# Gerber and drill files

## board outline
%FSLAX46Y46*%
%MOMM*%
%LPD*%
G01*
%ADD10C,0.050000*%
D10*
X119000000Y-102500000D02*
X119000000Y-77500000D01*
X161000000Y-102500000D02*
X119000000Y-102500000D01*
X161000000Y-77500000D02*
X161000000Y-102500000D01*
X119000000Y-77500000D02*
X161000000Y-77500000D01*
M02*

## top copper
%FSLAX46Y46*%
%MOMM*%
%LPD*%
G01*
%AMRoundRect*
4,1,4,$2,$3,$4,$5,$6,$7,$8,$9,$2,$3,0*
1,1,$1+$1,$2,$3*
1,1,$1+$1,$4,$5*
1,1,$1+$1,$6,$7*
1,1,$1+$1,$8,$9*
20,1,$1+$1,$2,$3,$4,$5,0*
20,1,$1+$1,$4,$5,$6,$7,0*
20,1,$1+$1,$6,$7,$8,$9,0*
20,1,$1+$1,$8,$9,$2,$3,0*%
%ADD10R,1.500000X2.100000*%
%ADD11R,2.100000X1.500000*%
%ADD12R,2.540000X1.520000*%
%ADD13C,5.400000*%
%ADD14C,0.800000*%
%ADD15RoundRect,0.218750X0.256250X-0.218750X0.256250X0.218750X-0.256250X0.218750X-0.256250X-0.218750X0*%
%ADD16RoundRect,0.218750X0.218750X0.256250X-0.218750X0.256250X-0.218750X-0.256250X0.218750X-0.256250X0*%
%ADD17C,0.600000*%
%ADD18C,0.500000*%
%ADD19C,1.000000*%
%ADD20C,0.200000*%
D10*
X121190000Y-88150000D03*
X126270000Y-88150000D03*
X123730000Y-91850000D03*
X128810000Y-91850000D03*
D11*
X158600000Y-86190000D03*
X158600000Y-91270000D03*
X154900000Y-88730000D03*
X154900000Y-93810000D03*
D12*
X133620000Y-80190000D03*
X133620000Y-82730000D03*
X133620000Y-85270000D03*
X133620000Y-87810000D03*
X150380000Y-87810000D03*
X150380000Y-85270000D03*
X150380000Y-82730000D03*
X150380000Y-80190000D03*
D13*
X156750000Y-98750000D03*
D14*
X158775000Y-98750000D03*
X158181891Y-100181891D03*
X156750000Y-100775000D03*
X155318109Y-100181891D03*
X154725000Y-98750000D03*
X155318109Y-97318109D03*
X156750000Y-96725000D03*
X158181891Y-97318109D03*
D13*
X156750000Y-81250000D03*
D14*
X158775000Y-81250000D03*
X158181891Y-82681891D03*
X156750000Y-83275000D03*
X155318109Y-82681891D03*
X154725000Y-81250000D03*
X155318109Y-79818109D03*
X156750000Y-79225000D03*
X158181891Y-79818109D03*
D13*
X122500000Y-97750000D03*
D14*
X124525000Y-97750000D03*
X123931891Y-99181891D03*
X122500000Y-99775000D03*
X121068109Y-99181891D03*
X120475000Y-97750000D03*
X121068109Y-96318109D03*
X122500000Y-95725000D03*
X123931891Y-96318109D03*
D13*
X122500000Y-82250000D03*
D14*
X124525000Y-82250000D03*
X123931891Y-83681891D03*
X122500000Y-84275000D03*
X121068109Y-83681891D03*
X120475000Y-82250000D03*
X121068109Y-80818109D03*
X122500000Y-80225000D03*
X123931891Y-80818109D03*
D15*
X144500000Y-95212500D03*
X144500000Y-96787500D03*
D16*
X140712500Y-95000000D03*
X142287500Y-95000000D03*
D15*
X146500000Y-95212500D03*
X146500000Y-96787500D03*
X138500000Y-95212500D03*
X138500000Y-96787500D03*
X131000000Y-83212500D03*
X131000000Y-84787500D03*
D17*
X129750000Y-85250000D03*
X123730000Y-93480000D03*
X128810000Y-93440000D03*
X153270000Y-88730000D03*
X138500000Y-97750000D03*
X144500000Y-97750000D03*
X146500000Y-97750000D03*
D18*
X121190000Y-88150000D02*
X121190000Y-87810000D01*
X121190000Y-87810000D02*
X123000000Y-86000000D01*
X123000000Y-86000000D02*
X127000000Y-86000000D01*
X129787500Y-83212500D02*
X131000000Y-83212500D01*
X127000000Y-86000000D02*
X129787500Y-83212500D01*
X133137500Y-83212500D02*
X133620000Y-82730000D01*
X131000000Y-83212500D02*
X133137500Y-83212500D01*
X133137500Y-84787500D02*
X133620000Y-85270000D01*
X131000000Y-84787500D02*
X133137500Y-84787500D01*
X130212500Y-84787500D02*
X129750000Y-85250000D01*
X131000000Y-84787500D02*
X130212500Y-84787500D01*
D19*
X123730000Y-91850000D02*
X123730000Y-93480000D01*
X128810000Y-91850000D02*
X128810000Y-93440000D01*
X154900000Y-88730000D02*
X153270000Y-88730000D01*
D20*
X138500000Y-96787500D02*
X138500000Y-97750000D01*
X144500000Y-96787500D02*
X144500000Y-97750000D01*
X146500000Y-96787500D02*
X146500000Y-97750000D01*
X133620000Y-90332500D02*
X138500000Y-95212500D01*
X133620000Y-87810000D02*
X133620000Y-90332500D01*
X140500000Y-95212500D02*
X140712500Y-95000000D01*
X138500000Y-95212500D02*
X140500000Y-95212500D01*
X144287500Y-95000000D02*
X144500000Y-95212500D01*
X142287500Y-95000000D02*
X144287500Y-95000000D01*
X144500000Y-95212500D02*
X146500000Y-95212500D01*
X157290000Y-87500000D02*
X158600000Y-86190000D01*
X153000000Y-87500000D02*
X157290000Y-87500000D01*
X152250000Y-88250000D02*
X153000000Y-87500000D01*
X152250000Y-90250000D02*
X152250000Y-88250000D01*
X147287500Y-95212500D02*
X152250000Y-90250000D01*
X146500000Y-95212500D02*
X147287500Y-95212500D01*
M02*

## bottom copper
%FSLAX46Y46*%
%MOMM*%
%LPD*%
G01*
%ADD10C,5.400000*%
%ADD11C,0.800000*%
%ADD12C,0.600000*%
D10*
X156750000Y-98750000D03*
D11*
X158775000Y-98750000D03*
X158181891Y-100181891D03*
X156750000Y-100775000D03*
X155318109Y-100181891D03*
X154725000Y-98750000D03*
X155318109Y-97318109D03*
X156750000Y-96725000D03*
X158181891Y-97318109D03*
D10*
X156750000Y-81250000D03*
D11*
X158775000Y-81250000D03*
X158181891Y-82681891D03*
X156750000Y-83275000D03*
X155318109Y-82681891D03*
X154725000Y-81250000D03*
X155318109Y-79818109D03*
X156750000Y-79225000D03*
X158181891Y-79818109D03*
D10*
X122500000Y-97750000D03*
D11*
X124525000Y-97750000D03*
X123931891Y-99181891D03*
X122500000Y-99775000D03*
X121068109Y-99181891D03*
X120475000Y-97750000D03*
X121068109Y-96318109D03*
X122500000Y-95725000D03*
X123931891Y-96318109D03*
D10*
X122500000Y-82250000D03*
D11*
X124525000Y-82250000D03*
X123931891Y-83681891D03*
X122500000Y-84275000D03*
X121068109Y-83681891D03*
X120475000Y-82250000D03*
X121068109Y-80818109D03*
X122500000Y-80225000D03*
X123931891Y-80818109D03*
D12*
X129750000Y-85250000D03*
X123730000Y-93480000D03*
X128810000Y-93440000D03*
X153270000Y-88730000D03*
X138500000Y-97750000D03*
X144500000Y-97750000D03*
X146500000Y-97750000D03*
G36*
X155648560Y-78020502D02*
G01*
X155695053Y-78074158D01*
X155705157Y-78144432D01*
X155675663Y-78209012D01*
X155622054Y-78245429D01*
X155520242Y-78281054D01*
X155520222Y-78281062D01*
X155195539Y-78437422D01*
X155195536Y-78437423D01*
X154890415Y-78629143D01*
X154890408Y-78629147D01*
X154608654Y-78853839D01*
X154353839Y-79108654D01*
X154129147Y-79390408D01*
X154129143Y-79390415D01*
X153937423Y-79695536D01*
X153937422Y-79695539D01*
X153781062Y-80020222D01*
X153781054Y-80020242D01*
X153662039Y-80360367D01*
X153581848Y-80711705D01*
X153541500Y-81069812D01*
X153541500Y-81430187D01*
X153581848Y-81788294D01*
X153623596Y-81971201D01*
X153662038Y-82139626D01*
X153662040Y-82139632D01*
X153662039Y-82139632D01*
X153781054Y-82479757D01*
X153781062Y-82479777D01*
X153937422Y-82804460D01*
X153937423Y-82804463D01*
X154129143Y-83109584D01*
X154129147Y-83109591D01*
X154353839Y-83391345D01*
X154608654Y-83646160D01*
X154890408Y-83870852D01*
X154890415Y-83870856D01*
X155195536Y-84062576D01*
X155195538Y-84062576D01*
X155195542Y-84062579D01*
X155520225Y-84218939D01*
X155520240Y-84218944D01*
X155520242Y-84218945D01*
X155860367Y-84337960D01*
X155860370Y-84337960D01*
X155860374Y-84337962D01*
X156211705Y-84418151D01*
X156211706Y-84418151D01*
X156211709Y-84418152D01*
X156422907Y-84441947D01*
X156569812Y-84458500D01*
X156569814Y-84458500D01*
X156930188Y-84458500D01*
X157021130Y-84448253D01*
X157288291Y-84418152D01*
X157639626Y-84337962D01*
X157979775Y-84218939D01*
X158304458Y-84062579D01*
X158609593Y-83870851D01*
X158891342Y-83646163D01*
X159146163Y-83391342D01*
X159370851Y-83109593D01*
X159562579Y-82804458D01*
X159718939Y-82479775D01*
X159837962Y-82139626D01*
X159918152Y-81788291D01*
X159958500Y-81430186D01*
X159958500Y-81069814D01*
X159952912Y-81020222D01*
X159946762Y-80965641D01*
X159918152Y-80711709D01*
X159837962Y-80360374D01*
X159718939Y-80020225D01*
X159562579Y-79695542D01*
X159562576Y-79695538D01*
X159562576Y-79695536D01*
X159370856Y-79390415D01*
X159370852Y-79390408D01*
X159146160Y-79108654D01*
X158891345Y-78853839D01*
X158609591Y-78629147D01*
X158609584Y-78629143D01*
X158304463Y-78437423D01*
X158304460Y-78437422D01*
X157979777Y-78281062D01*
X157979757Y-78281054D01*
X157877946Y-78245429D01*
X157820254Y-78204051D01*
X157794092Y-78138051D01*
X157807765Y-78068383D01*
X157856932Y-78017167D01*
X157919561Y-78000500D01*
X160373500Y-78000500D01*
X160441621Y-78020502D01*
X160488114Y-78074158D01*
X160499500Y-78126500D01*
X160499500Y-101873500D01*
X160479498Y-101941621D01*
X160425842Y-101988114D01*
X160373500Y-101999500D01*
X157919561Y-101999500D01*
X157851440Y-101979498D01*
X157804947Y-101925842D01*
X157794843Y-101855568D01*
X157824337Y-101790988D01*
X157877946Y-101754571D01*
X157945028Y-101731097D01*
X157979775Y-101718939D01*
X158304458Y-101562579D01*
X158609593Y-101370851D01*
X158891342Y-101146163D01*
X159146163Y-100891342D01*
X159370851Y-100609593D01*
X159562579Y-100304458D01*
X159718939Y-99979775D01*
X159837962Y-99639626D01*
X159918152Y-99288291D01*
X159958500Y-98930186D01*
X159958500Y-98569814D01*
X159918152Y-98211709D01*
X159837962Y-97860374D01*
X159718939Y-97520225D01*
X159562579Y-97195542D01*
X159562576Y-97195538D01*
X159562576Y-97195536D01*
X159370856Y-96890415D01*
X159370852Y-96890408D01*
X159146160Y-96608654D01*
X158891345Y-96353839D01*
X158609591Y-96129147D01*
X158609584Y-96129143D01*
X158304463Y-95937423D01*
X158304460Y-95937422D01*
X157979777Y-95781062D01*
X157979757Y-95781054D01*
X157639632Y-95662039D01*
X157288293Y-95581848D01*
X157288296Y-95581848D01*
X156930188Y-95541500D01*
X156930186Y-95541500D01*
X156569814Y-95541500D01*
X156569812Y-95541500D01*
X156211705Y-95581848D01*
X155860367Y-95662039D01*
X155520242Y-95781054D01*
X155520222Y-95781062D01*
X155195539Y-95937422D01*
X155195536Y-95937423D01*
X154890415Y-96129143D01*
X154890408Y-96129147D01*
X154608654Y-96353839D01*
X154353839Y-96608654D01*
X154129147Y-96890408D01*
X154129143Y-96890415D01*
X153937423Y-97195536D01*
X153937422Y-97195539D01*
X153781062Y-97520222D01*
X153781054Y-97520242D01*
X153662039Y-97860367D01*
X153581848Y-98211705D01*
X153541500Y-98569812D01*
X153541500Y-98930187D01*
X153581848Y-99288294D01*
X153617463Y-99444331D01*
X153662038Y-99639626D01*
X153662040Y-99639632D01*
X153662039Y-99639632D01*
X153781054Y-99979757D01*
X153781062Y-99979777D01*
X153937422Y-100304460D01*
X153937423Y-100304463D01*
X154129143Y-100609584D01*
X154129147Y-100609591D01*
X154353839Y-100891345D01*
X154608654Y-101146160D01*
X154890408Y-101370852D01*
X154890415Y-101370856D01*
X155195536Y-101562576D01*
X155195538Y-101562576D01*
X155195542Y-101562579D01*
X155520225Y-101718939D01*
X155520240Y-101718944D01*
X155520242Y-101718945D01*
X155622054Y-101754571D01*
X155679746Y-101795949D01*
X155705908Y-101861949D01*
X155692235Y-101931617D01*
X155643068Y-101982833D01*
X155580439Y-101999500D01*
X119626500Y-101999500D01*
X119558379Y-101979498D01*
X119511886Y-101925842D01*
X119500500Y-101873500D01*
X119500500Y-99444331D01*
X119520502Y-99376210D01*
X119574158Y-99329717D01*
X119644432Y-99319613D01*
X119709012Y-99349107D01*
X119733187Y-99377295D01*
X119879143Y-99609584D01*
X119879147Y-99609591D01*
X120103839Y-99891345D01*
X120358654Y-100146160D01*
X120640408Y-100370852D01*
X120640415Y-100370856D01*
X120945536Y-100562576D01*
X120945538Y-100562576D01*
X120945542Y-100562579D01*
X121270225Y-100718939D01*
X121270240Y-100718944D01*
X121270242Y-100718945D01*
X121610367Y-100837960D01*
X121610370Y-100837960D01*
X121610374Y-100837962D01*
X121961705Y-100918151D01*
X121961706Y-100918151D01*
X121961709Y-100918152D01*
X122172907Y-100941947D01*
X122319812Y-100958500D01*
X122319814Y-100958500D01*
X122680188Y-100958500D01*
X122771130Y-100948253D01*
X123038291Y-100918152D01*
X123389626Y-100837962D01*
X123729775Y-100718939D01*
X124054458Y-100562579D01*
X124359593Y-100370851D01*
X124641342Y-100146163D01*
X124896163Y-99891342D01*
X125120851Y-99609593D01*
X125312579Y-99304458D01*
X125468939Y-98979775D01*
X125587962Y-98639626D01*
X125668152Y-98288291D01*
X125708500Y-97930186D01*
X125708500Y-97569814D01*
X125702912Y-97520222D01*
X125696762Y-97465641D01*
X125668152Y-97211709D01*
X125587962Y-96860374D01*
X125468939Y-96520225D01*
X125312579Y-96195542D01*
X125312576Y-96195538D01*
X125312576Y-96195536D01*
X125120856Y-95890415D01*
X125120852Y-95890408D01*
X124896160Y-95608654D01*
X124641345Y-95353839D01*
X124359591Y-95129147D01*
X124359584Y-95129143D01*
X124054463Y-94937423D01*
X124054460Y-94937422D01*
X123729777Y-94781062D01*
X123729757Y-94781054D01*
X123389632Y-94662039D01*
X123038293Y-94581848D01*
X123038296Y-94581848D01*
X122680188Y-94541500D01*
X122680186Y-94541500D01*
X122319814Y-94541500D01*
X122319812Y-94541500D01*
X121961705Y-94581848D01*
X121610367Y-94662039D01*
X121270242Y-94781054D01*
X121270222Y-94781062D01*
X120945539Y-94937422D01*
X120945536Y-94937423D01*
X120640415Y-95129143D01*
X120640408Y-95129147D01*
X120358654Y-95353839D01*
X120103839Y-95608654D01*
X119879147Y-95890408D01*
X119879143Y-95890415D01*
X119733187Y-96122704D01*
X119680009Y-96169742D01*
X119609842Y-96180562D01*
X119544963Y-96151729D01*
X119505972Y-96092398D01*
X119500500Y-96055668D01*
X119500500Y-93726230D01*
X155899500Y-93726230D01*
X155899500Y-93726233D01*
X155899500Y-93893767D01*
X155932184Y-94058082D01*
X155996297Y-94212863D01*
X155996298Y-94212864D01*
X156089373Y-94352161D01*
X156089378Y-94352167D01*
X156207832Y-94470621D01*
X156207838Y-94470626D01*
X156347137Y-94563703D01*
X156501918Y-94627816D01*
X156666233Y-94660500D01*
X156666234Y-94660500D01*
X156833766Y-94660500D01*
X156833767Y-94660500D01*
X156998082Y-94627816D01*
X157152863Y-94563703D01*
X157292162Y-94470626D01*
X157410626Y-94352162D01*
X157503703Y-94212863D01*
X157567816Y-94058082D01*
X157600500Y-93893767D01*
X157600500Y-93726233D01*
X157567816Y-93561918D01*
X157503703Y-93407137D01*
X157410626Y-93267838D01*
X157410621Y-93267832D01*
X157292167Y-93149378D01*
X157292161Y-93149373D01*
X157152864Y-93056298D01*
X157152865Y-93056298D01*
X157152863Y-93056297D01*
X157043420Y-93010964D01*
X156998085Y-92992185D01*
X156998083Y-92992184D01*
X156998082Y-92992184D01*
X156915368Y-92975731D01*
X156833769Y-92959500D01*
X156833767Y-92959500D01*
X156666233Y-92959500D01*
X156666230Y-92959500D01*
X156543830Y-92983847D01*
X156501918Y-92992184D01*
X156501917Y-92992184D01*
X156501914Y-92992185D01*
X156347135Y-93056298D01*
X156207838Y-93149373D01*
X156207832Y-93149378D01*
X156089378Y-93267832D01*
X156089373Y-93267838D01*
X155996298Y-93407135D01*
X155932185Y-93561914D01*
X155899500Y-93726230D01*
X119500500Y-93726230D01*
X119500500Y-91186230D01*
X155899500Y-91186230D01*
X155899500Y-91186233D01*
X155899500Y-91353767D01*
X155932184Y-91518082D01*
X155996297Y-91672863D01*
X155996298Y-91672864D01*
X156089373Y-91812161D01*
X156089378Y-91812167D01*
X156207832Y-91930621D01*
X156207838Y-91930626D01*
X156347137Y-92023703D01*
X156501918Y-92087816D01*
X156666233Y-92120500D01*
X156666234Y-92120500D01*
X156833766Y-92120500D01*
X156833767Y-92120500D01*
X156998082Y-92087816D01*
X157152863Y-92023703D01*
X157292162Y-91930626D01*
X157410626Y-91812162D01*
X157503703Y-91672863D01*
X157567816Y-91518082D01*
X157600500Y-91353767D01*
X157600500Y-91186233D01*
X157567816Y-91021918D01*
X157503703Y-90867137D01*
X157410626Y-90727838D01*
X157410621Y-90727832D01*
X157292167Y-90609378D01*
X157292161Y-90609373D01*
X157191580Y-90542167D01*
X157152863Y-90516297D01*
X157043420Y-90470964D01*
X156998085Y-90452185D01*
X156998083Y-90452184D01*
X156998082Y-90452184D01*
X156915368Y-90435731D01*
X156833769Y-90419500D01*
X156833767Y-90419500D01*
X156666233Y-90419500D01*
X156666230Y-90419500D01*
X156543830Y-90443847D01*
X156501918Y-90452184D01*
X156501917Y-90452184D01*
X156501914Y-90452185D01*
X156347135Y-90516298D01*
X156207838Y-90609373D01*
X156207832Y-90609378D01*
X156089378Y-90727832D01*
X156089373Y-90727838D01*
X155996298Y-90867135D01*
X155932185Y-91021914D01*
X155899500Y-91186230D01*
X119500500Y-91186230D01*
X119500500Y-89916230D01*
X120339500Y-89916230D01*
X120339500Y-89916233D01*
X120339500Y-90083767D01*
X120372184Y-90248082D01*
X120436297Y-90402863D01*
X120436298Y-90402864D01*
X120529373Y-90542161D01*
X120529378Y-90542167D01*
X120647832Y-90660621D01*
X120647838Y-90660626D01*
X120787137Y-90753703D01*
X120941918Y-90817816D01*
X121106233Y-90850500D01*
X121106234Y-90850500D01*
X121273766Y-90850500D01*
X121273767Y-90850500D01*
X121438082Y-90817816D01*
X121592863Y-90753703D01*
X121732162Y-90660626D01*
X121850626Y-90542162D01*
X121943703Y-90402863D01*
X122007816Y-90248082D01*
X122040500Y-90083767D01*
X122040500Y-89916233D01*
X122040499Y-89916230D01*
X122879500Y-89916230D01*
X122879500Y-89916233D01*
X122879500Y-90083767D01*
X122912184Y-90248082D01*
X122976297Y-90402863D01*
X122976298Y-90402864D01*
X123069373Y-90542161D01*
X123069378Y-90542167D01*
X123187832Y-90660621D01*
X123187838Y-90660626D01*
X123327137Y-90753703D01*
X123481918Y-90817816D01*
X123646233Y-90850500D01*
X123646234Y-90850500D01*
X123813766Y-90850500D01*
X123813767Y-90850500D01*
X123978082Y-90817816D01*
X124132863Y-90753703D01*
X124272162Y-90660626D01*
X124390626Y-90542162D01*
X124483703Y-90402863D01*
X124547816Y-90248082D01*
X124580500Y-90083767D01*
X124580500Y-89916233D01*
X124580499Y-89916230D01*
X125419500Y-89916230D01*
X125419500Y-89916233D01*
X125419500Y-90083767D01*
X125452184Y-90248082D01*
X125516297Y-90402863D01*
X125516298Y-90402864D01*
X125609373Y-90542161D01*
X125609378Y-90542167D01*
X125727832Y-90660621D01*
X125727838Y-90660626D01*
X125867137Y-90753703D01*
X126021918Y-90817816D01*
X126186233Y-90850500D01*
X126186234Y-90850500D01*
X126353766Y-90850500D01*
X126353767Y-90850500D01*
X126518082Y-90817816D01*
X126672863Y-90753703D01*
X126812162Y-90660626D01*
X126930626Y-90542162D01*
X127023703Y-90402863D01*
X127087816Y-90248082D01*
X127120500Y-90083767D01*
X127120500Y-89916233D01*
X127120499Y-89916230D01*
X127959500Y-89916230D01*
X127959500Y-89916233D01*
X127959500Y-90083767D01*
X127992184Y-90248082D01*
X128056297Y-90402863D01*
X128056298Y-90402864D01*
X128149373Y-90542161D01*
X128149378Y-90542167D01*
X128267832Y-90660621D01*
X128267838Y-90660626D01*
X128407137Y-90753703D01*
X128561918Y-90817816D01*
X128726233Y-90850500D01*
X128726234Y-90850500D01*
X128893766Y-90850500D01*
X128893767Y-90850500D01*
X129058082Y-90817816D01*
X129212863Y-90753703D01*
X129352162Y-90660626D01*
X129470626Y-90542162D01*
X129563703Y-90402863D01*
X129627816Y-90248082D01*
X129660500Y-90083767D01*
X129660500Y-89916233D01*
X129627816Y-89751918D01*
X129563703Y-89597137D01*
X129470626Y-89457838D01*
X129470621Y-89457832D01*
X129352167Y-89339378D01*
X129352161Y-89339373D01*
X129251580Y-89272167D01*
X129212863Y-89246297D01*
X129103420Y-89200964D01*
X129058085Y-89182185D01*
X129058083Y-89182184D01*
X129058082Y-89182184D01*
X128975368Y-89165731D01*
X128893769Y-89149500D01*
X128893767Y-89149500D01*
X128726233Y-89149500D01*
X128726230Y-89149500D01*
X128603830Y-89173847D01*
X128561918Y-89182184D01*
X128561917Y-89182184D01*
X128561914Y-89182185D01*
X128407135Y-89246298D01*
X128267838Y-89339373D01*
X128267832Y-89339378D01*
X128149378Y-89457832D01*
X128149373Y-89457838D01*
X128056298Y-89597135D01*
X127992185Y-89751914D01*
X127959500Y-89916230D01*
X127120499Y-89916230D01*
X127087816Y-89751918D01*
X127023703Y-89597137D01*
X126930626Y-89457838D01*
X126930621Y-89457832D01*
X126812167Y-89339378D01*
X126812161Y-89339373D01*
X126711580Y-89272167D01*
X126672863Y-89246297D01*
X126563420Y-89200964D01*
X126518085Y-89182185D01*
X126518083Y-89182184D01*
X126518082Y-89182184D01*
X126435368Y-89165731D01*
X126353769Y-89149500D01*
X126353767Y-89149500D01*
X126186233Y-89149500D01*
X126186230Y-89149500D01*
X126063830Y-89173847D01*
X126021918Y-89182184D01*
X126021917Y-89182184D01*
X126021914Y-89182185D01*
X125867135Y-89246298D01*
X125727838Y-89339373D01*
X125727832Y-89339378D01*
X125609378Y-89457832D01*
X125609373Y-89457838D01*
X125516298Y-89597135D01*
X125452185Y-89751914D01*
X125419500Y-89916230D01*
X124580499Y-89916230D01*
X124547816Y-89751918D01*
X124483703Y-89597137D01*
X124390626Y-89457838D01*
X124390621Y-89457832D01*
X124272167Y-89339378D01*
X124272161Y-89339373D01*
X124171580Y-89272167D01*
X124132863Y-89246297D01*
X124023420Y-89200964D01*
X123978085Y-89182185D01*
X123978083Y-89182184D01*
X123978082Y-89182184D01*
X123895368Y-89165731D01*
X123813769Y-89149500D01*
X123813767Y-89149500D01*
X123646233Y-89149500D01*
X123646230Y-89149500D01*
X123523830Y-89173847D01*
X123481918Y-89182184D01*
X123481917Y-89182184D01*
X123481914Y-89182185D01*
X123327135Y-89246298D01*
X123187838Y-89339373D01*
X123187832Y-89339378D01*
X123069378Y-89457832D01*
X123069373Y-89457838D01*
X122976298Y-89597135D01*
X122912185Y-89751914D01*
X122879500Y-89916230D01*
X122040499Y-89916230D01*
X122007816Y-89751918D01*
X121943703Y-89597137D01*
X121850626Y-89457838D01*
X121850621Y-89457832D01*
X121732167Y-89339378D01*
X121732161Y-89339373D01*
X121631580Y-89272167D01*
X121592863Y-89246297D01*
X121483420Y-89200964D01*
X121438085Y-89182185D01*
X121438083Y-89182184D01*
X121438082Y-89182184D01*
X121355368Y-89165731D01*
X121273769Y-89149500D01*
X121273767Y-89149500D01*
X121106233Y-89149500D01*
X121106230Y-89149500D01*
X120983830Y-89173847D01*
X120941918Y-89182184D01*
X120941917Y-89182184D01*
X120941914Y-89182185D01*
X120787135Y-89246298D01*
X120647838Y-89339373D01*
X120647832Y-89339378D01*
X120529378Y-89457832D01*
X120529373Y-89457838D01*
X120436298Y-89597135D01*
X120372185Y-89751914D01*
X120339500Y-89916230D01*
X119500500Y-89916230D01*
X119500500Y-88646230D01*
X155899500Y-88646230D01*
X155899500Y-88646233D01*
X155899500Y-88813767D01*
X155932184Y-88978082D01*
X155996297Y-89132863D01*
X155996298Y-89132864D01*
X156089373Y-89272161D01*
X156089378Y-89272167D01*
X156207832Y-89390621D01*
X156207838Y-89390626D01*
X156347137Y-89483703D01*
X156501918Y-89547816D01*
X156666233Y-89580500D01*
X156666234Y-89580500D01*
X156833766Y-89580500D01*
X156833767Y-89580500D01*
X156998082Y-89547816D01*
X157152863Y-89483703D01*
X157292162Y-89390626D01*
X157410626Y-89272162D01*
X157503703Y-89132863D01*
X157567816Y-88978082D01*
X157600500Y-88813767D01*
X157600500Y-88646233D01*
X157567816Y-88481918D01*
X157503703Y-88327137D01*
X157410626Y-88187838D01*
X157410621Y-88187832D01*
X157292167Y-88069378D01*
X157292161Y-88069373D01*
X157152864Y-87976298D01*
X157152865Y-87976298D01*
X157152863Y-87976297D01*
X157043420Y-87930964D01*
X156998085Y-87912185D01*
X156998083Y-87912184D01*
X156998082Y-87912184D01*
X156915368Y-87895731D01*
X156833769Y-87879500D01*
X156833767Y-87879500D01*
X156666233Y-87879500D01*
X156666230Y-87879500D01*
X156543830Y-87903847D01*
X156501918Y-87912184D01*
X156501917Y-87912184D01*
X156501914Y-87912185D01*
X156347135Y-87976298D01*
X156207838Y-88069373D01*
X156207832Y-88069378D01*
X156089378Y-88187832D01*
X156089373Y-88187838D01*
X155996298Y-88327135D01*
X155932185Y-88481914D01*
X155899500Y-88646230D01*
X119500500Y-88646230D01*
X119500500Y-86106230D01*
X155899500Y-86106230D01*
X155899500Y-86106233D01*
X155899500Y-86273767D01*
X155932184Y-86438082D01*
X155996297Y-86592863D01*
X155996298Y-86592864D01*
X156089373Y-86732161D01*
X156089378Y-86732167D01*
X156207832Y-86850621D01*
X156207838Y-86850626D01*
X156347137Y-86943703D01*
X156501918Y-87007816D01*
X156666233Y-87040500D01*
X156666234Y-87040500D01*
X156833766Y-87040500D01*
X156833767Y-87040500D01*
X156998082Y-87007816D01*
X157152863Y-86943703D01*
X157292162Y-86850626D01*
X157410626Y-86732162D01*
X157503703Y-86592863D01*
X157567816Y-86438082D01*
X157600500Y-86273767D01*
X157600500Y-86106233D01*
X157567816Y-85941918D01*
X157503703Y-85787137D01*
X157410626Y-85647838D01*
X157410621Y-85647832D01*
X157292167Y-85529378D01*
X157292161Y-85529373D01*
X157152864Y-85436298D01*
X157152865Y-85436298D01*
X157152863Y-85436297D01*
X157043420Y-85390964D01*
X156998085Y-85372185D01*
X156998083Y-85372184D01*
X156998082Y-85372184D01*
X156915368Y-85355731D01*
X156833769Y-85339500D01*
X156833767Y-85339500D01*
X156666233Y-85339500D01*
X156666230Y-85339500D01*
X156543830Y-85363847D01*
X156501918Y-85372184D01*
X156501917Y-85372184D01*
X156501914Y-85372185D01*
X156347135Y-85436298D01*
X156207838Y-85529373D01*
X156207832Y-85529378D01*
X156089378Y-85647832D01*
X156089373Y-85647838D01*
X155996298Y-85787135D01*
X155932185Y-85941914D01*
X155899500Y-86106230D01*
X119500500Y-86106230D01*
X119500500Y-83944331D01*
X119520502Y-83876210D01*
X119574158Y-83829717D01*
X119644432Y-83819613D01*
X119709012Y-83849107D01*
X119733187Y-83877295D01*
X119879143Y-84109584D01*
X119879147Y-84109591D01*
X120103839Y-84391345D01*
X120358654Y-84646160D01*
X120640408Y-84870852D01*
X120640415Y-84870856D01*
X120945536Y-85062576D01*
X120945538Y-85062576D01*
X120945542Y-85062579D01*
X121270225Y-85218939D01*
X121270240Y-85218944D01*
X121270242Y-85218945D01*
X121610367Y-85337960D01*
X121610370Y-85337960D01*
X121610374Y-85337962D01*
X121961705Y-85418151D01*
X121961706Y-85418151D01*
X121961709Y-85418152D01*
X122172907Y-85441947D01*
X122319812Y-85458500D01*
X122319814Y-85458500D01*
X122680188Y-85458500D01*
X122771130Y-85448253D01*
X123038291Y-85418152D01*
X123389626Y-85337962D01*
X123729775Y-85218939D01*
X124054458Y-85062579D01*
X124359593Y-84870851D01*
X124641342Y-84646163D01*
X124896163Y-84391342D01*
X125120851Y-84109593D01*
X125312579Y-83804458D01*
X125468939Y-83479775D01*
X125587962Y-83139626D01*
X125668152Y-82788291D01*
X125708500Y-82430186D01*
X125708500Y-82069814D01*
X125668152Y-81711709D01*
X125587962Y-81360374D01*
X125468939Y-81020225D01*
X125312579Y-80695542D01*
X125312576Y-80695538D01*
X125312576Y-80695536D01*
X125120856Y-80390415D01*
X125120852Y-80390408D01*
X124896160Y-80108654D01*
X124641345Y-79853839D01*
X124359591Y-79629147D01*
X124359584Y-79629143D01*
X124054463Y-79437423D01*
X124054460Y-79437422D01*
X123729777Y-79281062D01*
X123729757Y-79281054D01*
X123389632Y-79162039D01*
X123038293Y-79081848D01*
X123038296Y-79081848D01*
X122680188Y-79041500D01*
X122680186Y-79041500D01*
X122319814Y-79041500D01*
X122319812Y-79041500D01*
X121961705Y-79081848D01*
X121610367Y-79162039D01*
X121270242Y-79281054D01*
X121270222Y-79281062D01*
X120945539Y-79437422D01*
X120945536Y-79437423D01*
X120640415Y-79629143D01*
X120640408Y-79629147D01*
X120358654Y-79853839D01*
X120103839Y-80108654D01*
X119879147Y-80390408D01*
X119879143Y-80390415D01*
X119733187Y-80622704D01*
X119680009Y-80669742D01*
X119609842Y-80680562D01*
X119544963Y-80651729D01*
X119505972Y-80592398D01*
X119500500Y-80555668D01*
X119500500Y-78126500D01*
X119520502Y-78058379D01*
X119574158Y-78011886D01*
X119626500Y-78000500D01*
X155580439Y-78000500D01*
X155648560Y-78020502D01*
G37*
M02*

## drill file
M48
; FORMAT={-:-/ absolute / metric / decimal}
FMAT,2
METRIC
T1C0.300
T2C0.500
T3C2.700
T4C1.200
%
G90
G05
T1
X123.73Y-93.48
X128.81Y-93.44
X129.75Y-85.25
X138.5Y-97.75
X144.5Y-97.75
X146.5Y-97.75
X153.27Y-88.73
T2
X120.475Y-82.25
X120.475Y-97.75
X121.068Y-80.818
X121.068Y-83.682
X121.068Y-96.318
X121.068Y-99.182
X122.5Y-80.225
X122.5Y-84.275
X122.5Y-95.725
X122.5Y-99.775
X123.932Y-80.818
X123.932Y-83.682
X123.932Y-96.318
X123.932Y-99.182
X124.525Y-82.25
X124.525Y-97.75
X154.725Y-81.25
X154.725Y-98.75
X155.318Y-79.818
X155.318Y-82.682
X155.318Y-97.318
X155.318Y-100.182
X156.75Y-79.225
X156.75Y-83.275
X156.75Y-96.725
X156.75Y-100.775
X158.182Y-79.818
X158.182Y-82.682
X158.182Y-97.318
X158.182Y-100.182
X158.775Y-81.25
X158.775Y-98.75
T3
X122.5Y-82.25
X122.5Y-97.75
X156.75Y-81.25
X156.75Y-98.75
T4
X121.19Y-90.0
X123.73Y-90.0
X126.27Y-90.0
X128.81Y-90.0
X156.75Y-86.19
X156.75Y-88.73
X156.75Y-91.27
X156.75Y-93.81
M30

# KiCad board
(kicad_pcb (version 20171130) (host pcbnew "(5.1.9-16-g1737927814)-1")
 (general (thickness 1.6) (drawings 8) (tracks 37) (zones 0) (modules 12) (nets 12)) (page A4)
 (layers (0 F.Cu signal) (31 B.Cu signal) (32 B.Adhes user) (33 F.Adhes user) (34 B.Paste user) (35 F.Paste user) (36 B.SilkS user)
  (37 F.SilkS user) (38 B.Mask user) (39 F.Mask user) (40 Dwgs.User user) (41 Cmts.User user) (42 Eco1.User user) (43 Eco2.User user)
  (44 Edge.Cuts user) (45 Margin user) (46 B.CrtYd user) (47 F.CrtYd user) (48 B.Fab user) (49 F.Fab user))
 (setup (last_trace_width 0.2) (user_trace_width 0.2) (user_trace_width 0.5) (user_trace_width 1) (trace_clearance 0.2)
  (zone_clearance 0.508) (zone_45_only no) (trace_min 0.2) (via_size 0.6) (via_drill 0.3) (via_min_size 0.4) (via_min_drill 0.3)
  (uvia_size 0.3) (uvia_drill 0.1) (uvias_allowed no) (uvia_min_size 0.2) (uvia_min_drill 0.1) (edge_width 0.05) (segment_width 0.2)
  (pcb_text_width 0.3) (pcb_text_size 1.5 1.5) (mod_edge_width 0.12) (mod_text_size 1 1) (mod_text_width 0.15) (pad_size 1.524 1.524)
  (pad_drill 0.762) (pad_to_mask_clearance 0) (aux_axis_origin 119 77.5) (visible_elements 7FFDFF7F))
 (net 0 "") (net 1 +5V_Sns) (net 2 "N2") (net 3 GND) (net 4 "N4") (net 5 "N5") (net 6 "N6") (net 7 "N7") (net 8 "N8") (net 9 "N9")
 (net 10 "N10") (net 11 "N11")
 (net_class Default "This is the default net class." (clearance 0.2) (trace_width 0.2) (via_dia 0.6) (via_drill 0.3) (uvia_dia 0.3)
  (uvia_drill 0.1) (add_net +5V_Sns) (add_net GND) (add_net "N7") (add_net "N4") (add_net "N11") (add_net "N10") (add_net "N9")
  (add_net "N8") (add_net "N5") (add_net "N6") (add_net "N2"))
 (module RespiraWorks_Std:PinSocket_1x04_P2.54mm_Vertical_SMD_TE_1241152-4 (layer F.Cu) (at 125 90 90)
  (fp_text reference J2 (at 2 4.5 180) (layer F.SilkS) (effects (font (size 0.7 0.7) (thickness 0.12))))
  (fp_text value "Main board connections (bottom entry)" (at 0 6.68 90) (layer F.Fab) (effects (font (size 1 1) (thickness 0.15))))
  (pad "" np_thru_hole circle (at 0 1.27 90) (size 1.2 1.2) (drill 1.2) (layers *.Cu *.Mask))
  (pad "" np_thru_hole circle (at 0 -1.27 90) (size 1.2 1.2) (drill 1.2) (layers *.Cu *.Mask))
  (pad "" np_thru_hole circle (at 0 -3.81 90) (size 1.2 1.2) (drill 1.2) (layers *.Cu *.Mask))
  (pad 1 smd rect (at 1.85 -3.81 90) (size 2.1 1.5) (layers F.Cu F.Paste F.Mask) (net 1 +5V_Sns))
  (pad 3 smd rect (at 1.85 1.27 90) (size 2.1 1.5) (layers F.Cu F.Paste F.Mask) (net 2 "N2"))
  (pad 2 smd rect (at -1.85 -1.27 90) (size 2.1 1.5) (layers F.Cu F.Paste F.Mask) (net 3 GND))
  (pad 4 smd rect (at -1.85 3.81 90) (size 2.1 1.5) (layers F.Cu F.Paste F.Mask) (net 3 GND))
  (pad "" np_thru_hole circle (at 0 3.81 90) (size 1.2 1.2) (drill 1.2) (layers *.Cu *.Mask)))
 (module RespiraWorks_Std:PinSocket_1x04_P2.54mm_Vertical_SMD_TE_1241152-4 (layer F.Cu) (at 156.75 90)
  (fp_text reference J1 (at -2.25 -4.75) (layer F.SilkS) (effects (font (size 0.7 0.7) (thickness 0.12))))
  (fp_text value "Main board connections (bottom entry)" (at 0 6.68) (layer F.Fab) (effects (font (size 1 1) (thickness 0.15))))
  (pad "" np_thru_hole circle (at 0 1.27) (size 1.2 1.2) (drill 1.2) (layers *.Cu *.Mask))
  (pad "" np_thru_hole circle (at 0 -1.27) (size 1.2 1.2) (drill 1.2) (layers *.Cu *.Mask))
  (pad "" np_thru_hole circle (at 0 -3.81) (size 1.2 1.2) (drill 1.2) (layers *.Cu *.Mask))
  (pad 1 smd rect (at 1.85 -3.81) (size 2.1 1.5) (layers F.Cu F.Paste F.Mask) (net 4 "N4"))
  (pad 3 smd rect (at 1.85 1.27) (size 2.1 1.5) (layers F.Cu F.Paste F.Mask) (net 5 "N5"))
  (pad 2 smd rect (at -1.85 -1.27) (size 2.1 1.5) (layers F.Cu F.Paste F.Mask) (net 3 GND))
  (pad 4 smd rect (at -1.85 3.81) (size 2.1 1.5) (layers F.Cu F.Paste F.Mask) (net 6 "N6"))
  (pad "" np_thru_hole circle (at 0 3.81) (size 1.2 1.2) (drill 1.2) (layers *.Cu *.Mask)))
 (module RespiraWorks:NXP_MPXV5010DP (layer F.Cu) (at 142 84)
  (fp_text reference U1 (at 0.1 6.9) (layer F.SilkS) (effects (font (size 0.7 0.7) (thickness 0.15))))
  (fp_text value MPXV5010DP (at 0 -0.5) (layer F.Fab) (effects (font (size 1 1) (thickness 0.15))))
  (pad 1 smd rect (at -8.38 -3.81) (size 2.54 1.52) (layers F.Cu F.Paste F.Mask))
  (pad 2 smd rect (at -8.38 -1.27) (size 2.54 1.52) (layers F.Cu F.Paste F.Mask) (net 1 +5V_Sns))
  (pad 3 smd rect (at -8.38 1.27) (size 2.54 1.52) (layers F.Cu F.Paste F.Mask) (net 3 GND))
  (pad 4 smd rect (at -8.38 3.81) (size 2.54 1.52) (layers F.Cu F.Paste F.Mask) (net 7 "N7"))
  (pad 5 smd rect (at 8.38 3.81) (size 2.54 1.52) (layers F.Cu F.Paste F.Mask))
  (pad 6 smd rect (at 8.38 1.27) (size 2.54 1.52) (layers F.Cu F.Paste F.Mask))
  (pad 7 smd rect (at 8.38 -1.27) (size 2.54 1.52) (layers F.Cu F.Paste F.Mask))
  (pad 8 smd rect (at 8.38 -3.81) (size 2.54 1.52) (layers F.Cu F.Paste F.Mask)))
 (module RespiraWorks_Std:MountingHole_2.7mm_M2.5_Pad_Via (layer F.Cu) (at 156.75 98.75)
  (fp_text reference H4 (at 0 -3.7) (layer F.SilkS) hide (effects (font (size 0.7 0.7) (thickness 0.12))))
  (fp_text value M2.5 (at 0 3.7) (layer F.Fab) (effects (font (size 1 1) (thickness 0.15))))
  (pad 1 thru_hole circle (at 0 0) (size 5.4 5.4) (drill 2.7) (layers *.Cu *.Mask) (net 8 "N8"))
  (pad 1 thru_hole circle (at 2.025 0) (size 0.8 0.8) (drill 0.5) (layers *.Cu *.Mask) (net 8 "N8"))
  (pad 1 thru_hole circle (at 1.431891 1.431891) (size 0.8 0.8) (drill 0.5) (layers *.Cu *.Mask) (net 8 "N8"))
  (pad 1 thru_hole circle (at 0 2.025) (size 0.8 0.8) (drill 0.5) (layers *.Cu *.Mask) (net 8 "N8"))
  (pad 1 thru_hole circle (at -1.431891 1.431891) (size 0.8 0.8) (drill 0.5) (layers *.Cu *.Mask) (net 8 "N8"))
  (pad 1 thru_hole circle (at -2.025 0) (size 0.8 0.8) (drill 0.5) (layers *.Cu *.Mask) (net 8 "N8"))
  (pad 1 thru_hole circle (at -1.431891 -1.431891) (size 0.8 0.8) (drill 0.5) (layers *.Cu *.Mask) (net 8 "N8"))
  (pad 1 thru_hole circle (at 0 -2.025) (size 0.8 0.8) (drill 0.5) (layers *.Cu *.Mask) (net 8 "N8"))
  (pad 1 thru_hole circle (at 1.431891 -1.431891) (size 0.8 0.8) (drill 0.5) (layers *.Cu *.Mask) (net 8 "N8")))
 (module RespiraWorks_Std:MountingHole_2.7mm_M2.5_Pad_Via (layer F.Cu) (at 156.75 81.25)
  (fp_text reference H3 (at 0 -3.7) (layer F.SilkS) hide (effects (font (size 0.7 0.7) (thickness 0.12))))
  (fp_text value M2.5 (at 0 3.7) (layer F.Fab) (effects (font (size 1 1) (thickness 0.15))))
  (pad 1 thru_hole circle (at 0 0) (size 5.4 5.4) (drill 2.7) (layers *.Cu *.Mask) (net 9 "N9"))
  (pad 1 thru_hole circle (at 2.025 0) (size 0.8 0.8) (drill 0.5) (layers *.Cu *.Mask) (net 9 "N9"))
  (pad 1 thru_hole circle (at 1.431891 1.431891) (size 0.8 0.8) (drill 0.5) (layers *.Cu *.Mask) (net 9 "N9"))
  (pad 1 thru_hole circle (at 0 2.025) (size 0.8 0.8) (drill 0.5) (layers *.Cu *.Mask) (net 9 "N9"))
  (pad 1 thru_hole circle (at -1.431891 1.431891) (size 0.8 0.8) (drill 0.5) (layers *.Cu *.Mask) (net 9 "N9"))
  (pad 1 thru_hole circle (at -2.025 0) (size 0.8 0.8) (drill 0.5) (layers *.Cu *.Mask) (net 9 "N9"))
  (pad 1 thru_hole circle (at -1.431891 -1.431891) (size 0.8 0.8) (drill 0.5) (layers *.Cu *.Mask) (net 9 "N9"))
  (pad 1 thru_hole circle (at 0 -2.025) (size 0.8 0.8) (drill 0.5) (layers *.Cu *.Mask) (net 9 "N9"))
  (pad 1 thru_hole circle (at 1.431891 -1.431891) (size 0.8 0.8) (drill 0.5) (layers *.Cu *.Mask) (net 9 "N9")))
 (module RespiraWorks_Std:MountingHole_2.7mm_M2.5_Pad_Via (layer F.Cu) (at 122.5 97.75)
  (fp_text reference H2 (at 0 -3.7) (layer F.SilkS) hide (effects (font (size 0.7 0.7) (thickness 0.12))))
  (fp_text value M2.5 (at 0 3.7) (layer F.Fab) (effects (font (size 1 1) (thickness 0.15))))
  (pad 1 thru_hole circle (at 0 0) (size 5.4 5.4) (drill 2.7) (layers *.Cu *.Mask) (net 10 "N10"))
  (pad 1 thru_hole circle (at 2.025 0) (size 0.8 0.8) (drill 0.5) (layers *.Cu *.Mask) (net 10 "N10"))
  (pad 1 thru_hole circle (at 1.431891 1.431891) (size 0.8 0.8) (drill 0.5) (layers *.Cu *.Mask) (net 10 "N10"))
  (pad 1 thru_hole circle (at 0 2.025) (size 0.8 0.8) (drill 0.5) (layers *.Cu *.Mask) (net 10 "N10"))
  (pad 1 thru_hole circle (at -1.431891 1.431891) (size 0.8 0.8) (drill 0.5) (layers *.Cu *.Mask) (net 10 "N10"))
  (pad 1 thru_hole circle (at -2.025 0) (size 0.8 0.8) (drill 0.5) (layers *.Cu *.Mask) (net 10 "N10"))
  (pad 1 thru_hole circle (at -1.431891 -1.431891) (size 0.8 0.8) (drill 0.5) (layers *.Cu *.Mask) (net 10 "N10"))
  (pad 1 thru_hole circle (at 0 -2.025) (size 0.8 0.8) (drill 0.5) (layers *.Cu *.Mask) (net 10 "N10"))
  (pad 1 thru_hole circle (at 1.431891 -1.431891) (size 0.8 0.8) (drill 0.5) (layers *.Cu *.Mask) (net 10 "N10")))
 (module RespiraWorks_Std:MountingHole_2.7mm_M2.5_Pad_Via (layer F.Cu) (at 122.5 82.25)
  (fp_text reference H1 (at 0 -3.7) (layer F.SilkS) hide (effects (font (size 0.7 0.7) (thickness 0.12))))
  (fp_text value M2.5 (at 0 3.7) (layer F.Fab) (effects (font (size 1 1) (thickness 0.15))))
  (pad 1 thru_hole circle (at 0 0) (size 5.4 5.4) (drill 2.7) (layers *.Cu *.Mask) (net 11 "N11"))
  (pad 1 thru_hole circle (at 2.025 0) (size 0.8 0.8) (drill 0.5) (layers *.Cu *.Mask) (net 11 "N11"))
  (pad 1 thru_hole circle (at 1.431891 1.431891) (size 0.8 0.8) (drill 0.5) (layers *.Cu *.Mask) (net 11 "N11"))
  (pad 1 thru_hole circle (at 0 2.025) (size 0.8 0.8) (drill 0.5) (layers *.Cu *.Mask) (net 11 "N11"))
  (pad 1 thru_hole circle (at -1.431891 1.431891) (size 0.8 0.8) (drill 0.5) (layers *.Cu *.Mask) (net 11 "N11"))
  (pad 1 thru_hole circle (at -2.025 0) (size 0.8 0.8) (drill 0.5) (layers *.Cu *.Mask) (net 11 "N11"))
  (pad 1 thru_hole circle (at -1.431891 -1.431891) (size 0.8 0.8) (drill 0.5) (layers *.Cu *.Mask) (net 11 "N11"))
  (pad 1 thru_hole circle (at 0 -2.025) (size 0.8 0.8) (drill 0.5) (layers *.Cu *.Mask) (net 11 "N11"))
  (pad 1 thru_hole circle (at 1.431891 -1.431891) (size 0.8 0.8) (drill 0.5) (layers *.Cu *.Mask) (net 11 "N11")))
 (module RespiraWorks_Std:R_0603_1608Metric (layer F.Cu) (at 144.5 96 90)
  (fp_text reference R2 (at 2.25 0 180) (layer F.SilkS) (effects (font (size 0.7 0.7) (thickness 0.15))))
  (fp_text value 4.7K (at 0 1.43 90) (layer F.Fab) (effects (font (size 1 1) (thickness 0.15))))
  (pad 2 smd roundrect (at 0.7875 0 90) (size 0.875 0.95) (layers F.Cu F.Paste F.Mask) (roundrect_rratio 0.25) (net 4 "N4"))
  (pad 1 smd roundrect (at -0.7875 0 90) (size 0.875 0.95) (layers F.Cu F.Paste F.Mask) (roundrect_rratio 0.25) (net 3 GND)))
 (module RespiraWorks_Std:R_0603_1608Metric (layer F.Cu) (at 141.5 95 180)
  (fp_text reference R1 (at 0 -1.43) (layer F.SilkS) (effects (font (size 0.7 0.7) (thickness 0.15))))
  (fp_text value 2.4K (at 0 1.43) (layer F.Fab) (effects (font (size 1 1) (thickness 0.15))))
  (pad 2 smd roundrect (at 0.7875 0 180) (size 0.875 0.95) (layers F.Cu F.Paste F.Mask) (roundrect_rratio 0.25) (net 7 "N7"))
  (pad 1 smd roundrect (at -0.7875 0 180) (size 0.875 0.95) (layers F.Cu F.Paste F.Mask) (roundrect_rratio 0.25) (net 4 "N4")))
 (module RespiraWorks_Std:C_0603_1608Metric (layer F.Cu) (at 146.5 96 90)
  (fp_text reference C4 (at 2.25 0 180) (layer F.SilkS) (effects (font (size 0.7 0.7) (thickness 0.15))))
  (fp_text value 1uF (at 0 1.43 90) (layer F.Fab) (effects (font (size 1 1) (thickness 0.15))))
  (pad 2 smd roundrect (at 0.7875 0 90) (size 0.875 0.95) (layers F.Cu F.Paste F.Mask) (roundrect_rratio 0.25) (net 4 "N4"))
  (pad 1 smd roundrect (at -0.7875 0 90) (size 0.875 0.95) (layers F.Cu F.Paste F.Mask) (roundrect_rratio 0.25) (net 3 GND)))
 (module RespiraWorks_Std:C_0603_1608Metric (layer F.Cu) (at 138.5 96 90)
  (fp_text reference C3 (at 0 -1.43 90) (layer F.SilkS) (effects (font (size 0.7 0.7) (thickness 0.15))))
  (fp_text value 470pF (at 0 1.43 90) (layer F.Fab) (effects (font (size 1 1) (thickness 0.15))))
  (pad 2 smd roundrect (at 0.7875 0 90) (size 0.875 0.95) (layers F.Cu F.Paste F.Mask) (roundrect_rratio 0.25) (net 7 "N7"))
  (pad 1 smd roundrect (at -0.7875 0 90) (size 0.875 0.95) (layers F.Cu F.Paste F.Mask) (roundrect_rratio 0.25) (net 3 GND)))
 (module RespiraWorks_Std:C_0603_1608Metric (layer F.Cu) (at 131 84 90)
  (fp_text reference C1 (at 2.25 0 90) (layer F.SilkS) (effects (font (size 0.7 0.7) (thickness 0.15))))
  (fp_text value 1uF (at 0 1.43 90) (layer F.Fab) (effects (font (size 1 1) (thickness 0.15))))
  (pad 2 smd roundrect (at 0.7875 0 90) (size 0.875 0.95) (layers F.Cu F.Paste F.Mask) (roundrect_rratio 0.25) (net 1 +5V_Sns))
  (pad 1 smd roundrect (at -0.7875 0 90) (size 0.875 0.95) (layers F.Cu F.Paste F.Mask) (roundrect_rratio 0.25) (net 3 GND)))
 (gr_line (start 119 102.5) (end 119 77.5) (layer Edge.Cuts) (width 0.05))
 (gr_line (start 161 102.5) (end 119 102.5) (layer Edge.Cuts) (width 0.05))
 (gr_line (start 161 77.5) (end 161 102.5) (layer Edge.Cuts) (width 0.05))
 (gr_line (start 119 77.5) (end 161 77.5) (layer Edge.Cuts) (width 0.05))
 (segment (start 121.19 88.15) (end 121.19 87.81) (width 0.5) (layer F.Cu) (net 1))
 (segment (start 121.19 87.81) (end 123 86) (width 0.5) (layer F.Cu) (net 1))
 (segment (start 123 86) (end 127 86) (width 0.5) (layer F.Cu) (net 1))
 (segment (start 129.7875 83.2125) (end 131 83.2125) (width 0.5) (layer F.Cu) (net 1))
 (segment (start 127 86) (end 129.7875 83.2125) (width 0.5) (layer F.Cu) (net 1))
 (segment (start 133.1375 83.2125) (end 133.62 82.73) (width 0.5) (layer F.Cu) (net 1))
 (segment (start 131 83.2125) (end 133.1375 83.2125) (width 0.5) (layer F.Cu) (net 1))
 (segment (start 133.1375 84.7875) (end 133.62 85.27) (width 0.5) (layer F.Cu) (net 3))
 (segment (start 131 84.7875) (end 133.1375 84.7875) (width 0.5) (layer F.Cu) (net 3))
 (via (at 129.75 85.25) (size 0.6) (drill 0.3) (layers F.Cu B.Cu) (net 3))
 (segment (start 130.2125 84.7875) (end 129.75 85.25) (width 0.5) (layer F.Cu) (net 3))
 (segment (start 131 84.7875) (end 130.2125 84.7875) (width 0.5) (layer F.Cu) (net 3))
 (segment (start 123.73 91.85) (end 123.73 93.48) (width 1) (layer F.Cu) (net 3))
 (via (at 123.73 93.48) (size 0.6) (drill 0.3) (layers F.Cu B.Cu) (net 3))
 (segment (start 128.81 91.85) (end 128.81 93.44) (width 1) (layer F.Cu) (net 3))
 (via (at 128.81 93.44) (size 0.6) (drill 0.3) (layers F.Cu B.Cu) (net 3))
 (segment (start 154.9 88.73) (end 153.27 88.73) (width 1) (layer F.Cu) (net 3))
 (via (at 153.27 88.73) (size 0.6) (drill 0.3) (layers F.Cu B.Cu) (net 3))
 (segment (start 138.5 96.7875) (end 138.5 97.75) (width 0.2) (layer F.Cu) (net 3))
 (via (at 138.5 97.75) (size 0.6) (drill 0.3) (layers F.Cu B.Cu) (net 3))
 (segment (start 144.5 96.7875) (end 144.5 97.75) (width 0.2) (layer F.Cu) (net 3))
 (via (at 144.5 97.75) (size 0.6) (drill 0.3) (layers F.Cu B.Cu) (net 3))
 (segment (start 146.5 96.7875) (end 146.5 97.75) (width 0.2) (layer F.Cu) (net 3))
 (via (at 146.5 97.75) (size 0.6) (drill 0.3) (layers F.Cu B.Cu) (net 3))
 (segment (start 133.62 90.3325) (end 138.5 95.2125) (width 0.2) (layer F.Cu) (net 7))
 (segment (start 133.62 87.81) (end 133.62 90.3325) (width 0.2) (layer F.Cu) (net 7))
 (segment (start 140.5 95.2125) (end 140.7125 95) (width 0.2) (layer F.Cu) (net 7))
 (segment (start 138.5 95.2125) (end 140.5 95.2125) (width 0.2) (layer F.Cu) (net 7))
 (segment (start 144.2875 95) (end 144.5 95.2125) (width 0.2) (layer F.Cu) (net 4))
 (segment (start 142.2875 95) (end 144.2875 95) (width 0.2) (layer F.Cu) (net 4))
 (segment (start 144.5 95.2125) (end 146.5 95.2125) (width 0.2) (layer F.Cu) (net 4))
 (segment (start 157.29 87.5) (end 158.6 86.19) (width 0.2) (layer F.Cu) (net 4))
 (segment (start 153 87.5) (end 157.29 87.5) (width 0.2) (layer F.Cu) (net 4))
 (segment (start 152.25 88.25) (end 153 87.5) (width 0.2) (layer F.Cu) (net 4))
 (segment (start 152.25 90.25) (end 152.25 88.25) (width 0.2) (layer F.Cu) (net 4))
 (segment (start 147.2875 95.2125) (end 152.25 90.25) (width 0.2) (layer F.Cu) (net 4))
 (segment (start 146.5 95.2125) (end 147.2875 95.2125) (width 0.2) (layer F.Cu) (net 4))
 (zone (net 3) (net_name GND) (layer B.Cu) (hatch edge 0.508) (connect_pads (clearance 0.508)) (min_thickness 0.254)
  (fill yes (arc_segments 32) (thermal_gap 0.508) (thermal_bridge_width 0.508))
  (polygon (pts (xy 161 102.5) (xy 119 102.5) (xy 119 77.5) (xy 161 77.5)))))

